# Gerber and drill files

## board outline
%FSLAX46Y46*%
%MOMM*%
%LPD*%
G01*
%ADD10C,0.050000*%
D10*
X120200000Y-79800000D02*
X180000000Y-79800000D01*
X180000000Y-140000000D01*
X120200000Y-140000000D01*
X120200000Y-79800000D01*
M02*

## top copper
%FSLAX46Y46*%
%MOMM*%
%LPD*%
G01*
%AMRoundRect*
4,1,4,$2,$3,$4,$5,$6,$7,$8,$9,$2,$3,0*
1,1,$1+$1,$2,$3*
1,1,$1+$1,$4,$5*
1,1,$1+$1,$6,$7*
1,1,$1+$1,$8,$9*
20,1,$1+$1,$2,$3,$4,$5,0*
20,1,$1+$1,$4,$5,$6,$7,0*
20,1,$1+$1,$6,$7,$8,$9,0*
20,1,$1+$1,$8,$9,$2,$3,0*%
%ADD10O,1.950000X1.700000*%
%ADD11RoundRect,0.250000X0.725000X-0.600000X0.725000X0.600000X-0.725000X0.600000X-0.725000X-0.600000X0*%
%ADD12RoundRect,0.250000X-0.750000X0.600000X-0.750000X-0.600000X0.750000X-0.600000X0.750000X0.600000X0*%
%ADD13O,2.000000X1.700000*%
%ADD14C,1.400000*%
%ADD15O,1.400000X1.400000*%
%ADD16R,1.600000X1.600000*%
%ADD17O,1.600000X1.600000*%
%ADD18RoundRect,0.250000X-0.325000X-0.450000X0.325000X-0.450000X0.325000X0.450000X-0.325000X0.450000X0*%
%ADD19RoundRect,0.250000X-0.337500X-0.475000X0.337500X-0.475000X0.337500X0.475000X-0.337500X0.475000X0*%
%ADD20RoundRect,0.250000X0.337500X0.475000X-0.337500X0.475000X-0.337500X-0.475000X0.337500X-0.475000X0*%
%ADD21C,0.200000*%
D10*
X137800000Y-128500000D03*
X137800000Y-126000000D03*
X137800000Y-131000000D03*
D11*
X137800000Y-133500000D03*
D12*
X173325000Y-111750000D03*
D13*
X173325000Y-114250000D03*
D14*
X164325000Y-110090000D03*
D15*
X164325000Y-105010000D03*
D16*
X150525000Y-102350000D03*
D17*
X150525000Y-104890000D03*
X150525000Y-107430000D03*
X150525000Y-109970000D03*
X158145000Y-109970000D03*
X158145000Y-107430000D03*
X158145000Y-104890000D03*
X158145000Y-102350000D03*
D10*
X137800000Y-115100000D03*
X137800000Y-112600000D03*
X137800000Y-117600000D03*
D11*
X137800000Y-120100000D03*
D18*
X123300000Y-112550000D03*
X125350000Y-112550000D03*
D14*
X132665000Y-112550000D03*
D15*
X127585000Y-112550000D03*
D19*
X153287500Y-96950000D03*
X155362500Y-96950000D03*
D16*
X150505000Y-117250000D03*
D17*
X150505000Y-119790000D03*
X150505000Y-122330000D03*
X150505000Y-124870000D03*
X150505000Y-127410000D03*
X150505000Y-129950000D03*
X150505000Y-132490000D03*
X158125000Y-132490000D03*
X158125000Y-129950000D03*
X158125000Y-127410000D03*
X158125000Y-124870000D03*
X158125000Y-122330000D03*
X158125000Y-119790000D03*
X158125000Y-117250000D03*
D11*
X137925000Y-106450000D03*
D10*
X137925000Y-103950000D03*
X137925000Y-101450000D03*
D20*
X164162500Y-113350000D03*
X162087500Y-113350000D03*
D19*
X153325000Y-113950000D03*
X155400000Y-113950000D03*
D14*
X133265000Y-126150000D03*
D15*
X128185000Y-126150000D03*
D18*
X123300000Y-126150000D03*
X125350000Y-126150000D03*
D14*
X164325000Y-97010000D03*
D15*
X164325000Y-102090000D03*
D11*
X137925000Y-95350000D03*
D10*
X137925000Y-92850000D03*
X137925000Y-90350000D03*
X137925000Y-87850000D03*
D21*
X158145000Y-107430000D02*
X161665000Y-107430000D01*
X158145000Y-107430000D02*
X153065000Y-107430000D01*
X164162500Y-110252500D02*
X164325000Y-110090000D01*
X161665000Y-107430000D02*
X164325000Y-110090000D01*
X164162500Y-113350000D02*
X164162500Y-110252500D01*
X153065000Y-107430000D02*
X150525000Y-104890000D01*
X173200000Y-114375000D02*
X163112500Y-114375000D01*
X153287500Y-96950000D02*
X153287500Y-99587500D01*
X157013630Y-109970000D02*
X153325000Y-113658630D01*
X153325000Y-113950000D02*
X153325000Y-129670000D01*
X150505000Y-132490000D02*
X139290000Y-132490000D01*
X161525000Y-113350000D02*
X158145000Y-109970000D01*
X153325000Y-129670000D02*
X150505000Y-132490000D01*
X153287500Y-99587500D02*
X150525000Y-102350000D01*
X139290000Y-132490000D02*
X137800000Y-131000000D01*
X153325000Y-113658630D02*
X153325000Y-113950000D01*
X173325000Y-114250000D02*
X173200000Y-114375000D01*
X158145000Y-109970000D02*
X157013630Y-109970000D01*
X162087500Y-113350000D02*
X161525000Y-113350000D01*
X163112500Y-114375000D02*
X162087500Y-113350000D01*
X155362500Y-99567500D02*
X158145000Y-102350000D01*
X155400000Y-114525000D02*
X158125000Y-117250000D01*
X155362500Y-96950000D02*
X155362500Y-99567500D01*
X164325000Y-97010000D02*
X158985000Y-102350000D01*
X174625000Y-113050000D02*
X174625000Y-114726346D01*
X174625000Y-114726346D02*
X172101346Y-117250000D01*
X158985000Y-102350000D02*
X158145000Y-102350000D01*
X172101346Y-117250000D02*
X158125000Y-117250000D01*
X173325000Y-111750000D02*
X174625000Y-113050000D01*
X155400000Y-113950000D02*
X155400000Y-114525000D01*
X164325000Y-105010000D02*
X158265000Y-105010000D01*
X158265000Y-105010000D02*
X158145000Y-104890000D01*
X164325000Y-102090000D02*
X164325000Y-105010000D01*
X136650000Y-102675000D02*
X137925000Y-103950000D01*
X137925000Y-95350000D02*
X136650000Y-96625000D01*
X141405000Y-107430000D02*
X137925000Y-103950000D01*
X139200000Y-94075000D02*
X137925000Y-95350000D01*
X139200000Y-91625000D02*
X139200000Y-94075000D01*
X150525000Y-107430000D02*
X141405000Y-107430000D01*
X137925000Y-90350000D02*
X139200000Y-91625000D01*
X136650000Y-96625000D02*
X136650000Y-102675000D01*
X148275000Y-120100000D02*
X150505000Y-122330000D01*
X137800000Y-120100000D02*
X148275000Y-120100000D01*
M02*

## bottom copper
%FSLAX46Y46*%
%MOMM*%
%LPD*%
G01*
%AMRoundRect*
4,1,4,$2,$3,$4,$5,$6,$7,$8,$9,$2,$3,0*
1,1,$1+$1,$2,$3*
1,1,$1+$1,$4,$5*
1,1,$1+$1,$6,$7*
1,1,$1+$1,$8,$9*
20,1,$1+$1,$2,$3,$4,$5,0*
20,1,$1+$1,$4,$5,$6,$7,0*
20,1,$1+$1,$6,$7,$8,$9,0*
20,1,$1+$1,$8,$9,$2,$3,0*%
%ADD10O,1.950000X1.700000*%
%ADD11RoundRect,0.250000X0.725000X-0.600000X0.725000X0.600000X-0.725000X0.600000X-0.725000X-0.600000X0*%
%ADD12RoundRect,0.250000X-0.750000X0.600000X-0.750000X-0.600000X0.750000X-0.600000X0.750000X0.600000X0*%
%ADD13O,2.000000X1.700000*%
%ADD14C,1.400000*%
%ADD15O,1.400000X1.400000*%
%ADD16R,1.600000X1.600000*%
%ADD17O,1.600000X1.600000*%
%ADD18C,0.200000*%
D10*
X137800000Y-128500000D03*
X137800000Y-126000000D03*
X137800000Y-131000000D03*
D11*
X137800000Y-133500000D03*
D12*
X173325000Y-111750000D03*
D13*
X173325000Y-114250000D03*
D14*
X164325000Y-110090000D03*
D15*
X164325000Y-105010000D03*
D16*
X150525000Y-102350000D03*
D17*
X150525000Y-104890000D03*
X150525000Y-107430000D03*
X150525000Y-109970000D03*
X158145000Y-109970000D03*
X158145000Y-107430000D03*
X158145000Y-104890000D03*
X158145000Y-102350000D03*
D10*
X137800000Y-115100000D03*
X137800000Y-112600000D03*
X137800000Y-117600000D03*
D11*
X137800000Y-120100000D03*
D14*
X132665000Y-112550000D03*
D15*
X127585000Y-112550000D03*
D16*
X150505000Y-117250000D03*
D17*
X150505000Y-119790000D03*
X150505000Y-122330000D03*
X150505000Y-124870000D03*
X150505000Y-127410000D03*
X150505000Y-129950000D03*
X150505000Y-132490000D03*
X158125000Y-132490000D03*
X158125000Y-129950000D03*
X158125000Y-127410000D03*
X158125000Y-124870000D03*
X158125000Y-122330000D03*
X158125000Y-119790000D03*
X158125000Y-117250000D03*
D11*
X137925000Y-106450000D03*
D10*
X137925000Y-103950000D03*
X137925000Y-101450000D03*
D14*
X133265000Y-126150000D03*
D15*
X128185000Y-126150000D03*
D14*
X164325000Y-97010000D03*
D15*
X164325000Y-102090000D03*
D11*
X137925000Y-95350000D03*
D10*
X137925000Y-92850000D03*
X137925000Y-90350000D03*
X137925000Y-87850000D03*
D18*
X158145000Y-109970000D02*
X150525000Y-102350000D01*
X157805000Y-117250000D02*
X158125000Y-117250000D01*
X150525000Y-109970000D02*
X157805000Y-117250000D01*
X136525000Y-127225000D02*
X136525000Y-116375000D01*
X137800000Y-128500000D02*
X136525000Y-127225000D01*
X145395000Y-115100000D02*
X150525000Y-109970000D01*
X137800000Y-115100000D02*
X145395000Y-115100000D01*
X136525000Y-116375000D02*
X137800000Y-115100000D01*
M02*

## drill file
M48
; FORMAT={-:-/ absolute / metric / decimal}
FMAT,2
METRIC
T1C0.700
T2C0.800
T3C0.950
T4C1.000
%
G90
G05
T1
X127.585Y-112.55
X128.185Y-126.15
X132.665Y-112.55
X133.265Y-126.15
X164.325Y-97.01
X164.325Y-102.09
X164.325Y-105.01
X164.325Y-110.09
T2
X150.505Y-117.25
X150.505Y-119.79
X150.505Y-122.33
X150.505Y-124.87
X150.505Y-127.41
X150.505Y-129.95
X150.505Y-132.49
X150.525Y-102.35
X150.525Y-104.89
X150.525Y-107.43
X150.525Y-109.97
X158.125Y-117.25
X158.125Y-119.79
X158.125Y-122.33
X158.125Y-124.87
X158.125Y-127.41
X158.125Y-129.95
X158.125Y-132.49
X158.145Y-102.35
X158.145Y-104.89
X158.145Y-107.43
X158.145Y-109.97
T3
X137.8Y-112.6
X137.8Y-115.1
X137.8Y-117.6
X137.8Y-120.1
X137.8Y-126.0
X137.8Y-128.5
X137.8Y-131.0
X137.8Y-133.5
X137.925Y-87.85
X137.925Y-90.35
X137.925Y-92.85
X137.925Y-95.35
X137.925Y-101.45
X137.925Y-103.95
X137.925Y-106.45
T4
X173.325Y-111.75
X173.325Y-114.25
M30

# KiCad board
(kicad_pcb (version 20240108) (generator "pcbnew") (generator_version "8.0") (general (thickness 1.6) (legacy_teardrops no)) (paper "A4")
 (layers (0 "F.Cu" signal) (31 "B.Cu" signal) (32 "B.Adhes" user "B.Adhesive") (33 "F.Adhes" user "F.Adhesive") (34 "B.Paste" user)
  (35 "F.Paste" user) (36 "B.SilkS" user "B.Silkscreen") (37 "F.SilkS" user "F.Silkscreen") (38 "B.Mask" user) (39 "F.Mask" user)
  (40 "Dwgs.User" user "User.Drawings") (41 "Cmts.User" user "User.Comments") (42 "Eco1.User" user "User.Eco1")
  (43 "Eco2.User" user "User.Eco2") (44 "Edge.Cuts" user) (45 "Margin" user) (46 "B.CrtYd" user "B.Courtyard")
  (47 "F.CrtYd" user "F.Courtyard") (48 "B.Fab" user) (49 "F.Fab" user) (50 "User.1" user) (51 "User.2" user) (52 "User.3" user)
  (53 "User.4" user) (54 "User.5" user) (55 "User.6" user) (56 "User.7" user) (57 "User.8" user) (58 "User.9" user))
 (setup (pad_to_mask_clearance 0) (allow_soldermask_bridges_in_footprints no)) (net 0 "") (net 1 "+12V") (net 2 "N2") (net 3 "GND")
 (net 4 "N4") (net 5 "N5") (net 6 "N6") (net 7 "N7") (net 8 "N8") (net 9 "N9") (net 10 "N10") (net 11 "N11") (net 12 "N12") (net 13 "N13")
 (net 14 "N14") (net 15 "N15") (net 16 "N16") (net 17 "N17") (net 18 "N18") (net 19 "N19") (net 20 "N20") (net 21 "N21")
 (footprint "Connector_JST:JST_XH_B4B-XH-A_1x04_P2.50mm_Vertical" (layer "F.Cu") (at 137.8 133.5 90)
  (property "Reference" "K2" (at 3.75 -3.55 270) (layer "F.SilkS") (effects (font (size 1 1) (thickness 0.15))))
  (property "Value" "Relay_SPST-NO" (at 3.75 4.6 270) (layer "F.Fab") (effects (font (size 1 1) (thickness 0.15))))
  (pad "13" thru_hole oval (at 5 0 90) (size 1.7 1.95) (drill 0.95) (layers "*.Cu" "*.Mask") (remove_unused_layers no) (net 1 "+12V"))
  (pad "14" thru_hole oval (at 7.5 0 90) (size 1.7 1.95) (drill 0.95) (layers "*.Cu" "*.Mask") (remove_unused_layers no) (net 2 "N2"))
  (pad "A1" thru_hole oval (at 2.5 0 90) (size 1.7 1.95) (drill 0.95) (layers "*.Cu" "*.Mask") (remove_unused_layers no) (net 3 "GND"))
  (pad "A2" thru_hole roundrect (at 0 0 90) (size 1.7 1.95) (drill 0.95) (layers "*.Cu" "*.Mask") (remove_unused_layers no)
   (roundrect_rratio 0.147059) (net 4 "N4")))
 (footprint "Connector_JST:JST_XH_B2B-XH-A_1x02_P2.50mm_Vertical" (layer "F.Cu") (at 173.325 111.75 -90)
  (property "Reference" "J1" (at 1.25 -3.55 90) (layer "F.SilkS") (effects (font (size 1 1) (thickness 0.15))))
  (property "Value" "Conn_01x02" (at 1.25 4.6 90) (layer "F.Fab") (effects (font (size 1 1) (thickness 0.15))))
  (pad "1" thru_hole roundrect (at 0 0 270) (size 1.7 2) (drill 1) (layers "*.Cu" "*.Mask") (remove_unused_layers no)
   (roundrect_rratio 0.147059) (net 1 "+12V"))
  (pad "2" thru_hole oval (at 2.5 0 270) (size 1.7 2) (drill 1) (layers "*.Cu" "*.Mask") (remove_unused_layers no) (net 3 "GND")))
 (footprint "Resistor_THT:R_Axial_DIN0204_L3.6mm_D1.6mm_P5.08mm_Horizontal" (layer "F.Cu") (at 164.325 110.09 90)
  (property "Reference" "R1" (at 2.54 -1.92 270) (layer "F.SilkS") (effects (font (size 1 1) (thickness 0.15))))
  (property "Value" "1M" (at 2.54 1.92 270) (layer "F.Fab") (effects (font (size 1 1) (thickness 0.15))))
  (pad "1" thru_hole circle (at 0 0 90) (size 1.4 1.4) (drill 0.7) (layers "*.Cu" "*.Mask") (remove_unused_layers no) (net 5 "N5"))
  (pad "2" thru_hole oval (at 5.08 0 90) (size 1.4 1.4) (drill 0.7) (layers "*.Cu" "*.Mask") (remove_unused_layers no) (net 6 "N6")))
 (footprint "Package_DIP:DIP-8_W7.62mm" (layer "F.Cu") (at 150.525 102.35)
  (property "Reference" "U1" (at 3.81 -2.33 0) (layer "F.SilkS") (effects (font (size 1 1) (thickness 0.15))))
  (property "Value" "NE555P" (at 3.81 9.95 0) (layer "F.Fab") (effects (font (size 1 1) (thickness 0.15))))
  (pad "1" thru_hole rect (at 0 0) (size 1.6 1.6) (drill 0.8) (layers "*.Cu" "*.Mask") (remove_unused_layers no) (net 3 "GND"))
  (pad "2" thru_hole oval (at 0 2.54) (size 1.6 1.6) (drill 0.8) (layers "*.Cu" "*.Mask") (remove_unused_layers no) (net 5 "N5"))
  (pad "3" thru_hole oval (at 0 5.08) (size 1.6 1.6) (drill 0.8) (layers "*.Cu" "*.Mask") (remove_unused_layers no) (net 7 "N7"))
  (pad "4" thru_hole oval (at 0 7.62) (size 1.6 1.6) (drill 0.8) (layers "*.Cu" "*.Mask") (remove_unused_layers no) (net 1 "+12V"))
  (pad "5" thru_hole oval (at 7.62 7.62) (size 1.6 1.6) (drill 0.8) (layers "*.Cu" "*.Mask") (remove_unused_layers no) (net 3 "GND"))
  (pad "6" thru_hole oval (at 7.62 5.08) (size 1.6 1.6) (drill 0.8) (layers "*.Cu" "*.Mask") (remove_unused_layers no) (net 5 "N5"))
  (pad "7" thru_hole oval (at 7.62 2.54) (size 1.6 1.6) (drill 0.8) (layers "*.Cu" "*.Mask") (remove_unused_layers no) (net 6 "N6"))
  (pad "8" thru_hole oval (at 7.62 0) (size 1.6 1.6) (drill 0.8) (layers "*.Cu" "*.Mask") (remove_unused_layers no) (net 1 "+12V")))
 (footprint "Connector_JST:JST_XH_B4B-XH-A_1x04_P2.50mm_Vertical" (layer "F.Cu") (at 137.8 120.1 90)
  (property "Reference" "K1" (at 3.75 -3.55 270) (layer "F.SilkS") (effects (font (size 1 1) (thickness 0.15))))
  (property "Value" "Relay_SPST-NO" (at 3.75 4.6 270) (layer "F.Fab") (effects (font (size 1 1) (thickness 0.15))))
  (pad "13" thru_hole oval (at 5 0 90) (size 1.7 1.95) (drill 0.95) (layers "*.Cu" "*.Mask") (remove_unused_layers no) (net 1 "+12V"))
  (pad "14" thru_hole oval (at 7.5 0 90) (size 1.7 1.95) (drill 0.95) (layers "*.Cu" "*.Mask") (remove_unused_layers no) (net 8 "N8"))
  (pad "A1" thru_hole oval (at 2.5 0 90) (size 1.7 1.95) (drill 0.95) (layers "*.Cu" "*.Mask") (remove_unused_layers no) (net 3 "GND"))
  (pad "A2" thru_hole roundrect (at 0 0 90) (size 1.7 1.95) (drill 0.95) (layers "*.Cu" "*.Mask") (remove_unused_layers no)
   (roundrect_rratio 0.147059) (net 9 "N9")))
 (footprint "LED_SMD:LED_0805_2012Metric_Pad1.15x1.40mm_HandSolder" (layer "F.Cu") (at 124.325 112.55)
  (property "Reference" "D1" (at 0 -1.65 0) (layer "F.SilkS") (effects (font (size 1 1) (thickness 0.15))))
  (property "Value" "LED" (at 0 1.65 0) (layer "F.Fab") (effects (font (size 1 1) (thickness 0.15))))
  (pad "1" smd roundrect (at -1.025 0) (size 1.15 1.4) (layers "F.Cu" "F.Paste" "F.Mask") (roundrect_rratio 0.217391) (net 3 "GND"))
  (pad "2" smd roundrect (at 1.025 0) (size 1.15 1.4) (layers "F.Cu" "F.Paste" "F.Mask") (roundrect_rratio 0.217391) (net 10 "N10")))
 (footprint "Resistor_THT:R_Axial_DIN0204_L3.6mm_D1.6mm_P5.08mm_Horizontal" (layer "F.Cu") (at 132.665 112.55 180)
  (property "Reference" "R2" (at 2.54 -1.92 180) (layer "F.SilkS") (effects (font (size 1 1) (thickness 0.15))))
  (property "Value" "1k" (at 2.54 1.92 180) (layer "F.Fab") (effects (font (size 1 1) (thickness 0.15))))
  (pad "1" thru_hole circle (at 0 0 180) (size 1.4 1.4) (drill 0.7) (layers "*.Cu" "*.Mask") (remove_unused_layers no) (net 8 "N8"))
  (pad "2" thru_hole oval (at 5.08 0 180) (size 1.4 1.4) (drill 0.7) (layers "*.Cu" "*.Mask") (remove_unused_layers no) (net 10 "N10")))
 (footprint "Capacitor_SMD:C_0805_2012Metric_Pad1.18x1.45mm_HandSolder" (layer "F.Cu") (at 154.325 96.95)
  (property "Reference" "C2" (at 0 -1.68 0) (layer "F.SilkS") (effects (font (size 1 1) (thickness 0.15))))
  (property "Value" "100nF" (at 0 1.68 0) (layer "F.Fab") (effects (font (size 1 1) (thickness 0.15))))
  (pad "1" smd roundrect (at -1.0375 0) (size 1.175 1.45) (layers "F.Cu" "F.Paste" "F.Mask") (roundrect_rratio 0.212766) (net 3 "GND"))
  (pad "2" smd roundrect (at 1.0375 0) (size 1.175 1.45) (layers "F.Cu" "F.Paste" "F.Mask") (roundrect_rratio 0.212766) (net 1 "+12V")))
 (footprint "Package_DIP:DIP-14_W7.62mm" (layer "F.Cu") (at 150.505 117.25)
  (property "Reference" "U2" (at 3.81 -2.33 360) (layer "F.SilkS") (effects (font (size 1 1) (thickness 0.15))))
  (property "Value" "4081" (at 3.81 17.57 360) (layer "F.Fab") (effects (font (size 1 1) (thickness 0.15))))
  (pad "1" thru_hole rect (at 0 0) (size 1.6 1.6) (drill 0.8) (layers "*.Cu" "*.Mask") (remove_unused_layers no) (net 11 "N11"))
  (pad "2" thru_hole oval (at 0 2.54) (size 1.6 1.6) (drill 0.8) (layers "*.Cu" "*.Mask") (remove_unused_layers no) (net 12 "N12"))
  (pad "3" thru_hole oval (at 0 5.08) (size 1.6 1.6) (drill 0.8) (layers "*.Cu" "*.Mask") (remove_unused_layers no) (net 9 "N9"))
  (pad "4" thru_hole oval (at 0 7.62) (size 1.6 1.6) (drill 0.8) (layers "*.Cu" "*.Mask") (remove_unused_layers no) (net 4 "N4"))
  (pad "5" thru_hole oval (at 0 10.16) (size 1.6 1.6) (drill 0.8) (layers "*.Cu" "*.Mask") (remove_unused_layers no) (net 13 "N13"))
  (pad "6" thru_hole oval (at 0 12.7) (size 1.6 1.6) (drill 0.8) (layers "*.Cu" "*.Mask") (remove_unused_layers no) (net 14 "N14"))
  (pad "7" thru_hole oval (at 0 15.24) (size 1.6 1.6) (drill 0.8) (layers "*.Cu" "*.Mask") (remove_unused_layers no) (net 3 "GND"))
  (pad "8" thru_hole oval (at 7.62 15.24) (size 1.6 1.6) (drill 0.8) (layers "*.Cu" "*.Mask") (remove_unused_layers no) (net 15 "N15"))
  (pad "9" thru_hole oval (at 7.62 12.7) (size 1.6 1.6) (drill 0.8) (layers "*.Cu" "*.Mask") (remove_unused_layers no) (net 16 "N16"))
  (pad "10" thru_hole oval (at 7.62 10.16) (size 1.6 1.6) (drill 0.8) (layers "*.Cu" "*.Mask") (remove_unused_layers no) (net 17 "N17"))
  (pad "11" thru_hole oval (at 7.62 7.62) (size 1.6 1.6) (drill 0.8) (layers "*.Cu" "*.Mask") (remove_unused_layers no) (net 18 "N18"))
  (pad "12" thru_hole oval (at 7.62 5.08) (size 1.6 1.6) (drill 0.8) (layers "*.Cu" "*.Mask") (remove_unused_layers no) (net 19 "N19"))
  (pad "13" thru_hole oval (at 7.62 2.54) (size 1.6 1.6) (drill 0.8) (layers "*.Cu" "*.Mask") (remove_unused_layers no) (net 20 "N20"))
  (pad "14" thru_hole oval (at 7.62 0) (size 1.6 1.6) (drill 0.8) (layers "*.Cu" "*.Mask") (remove_unused_layers no) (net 1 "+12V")))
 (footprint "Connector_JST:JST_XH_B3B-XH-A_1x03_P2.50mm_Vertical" (layer "F.Cu") (at 137.925 106.45 90)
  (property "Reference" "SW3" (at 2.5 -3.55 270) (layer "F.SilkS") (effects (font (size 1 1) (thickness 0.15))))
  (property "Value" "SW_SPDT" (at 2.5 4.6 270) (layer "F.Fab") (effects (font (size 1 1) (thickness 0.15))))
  (pad "1" thru_hole roundrect (at 0 0 90) (size 1.7 1.95) (drill 0.95) (layers "*.Cu" "*.Mask") (remove_unused_layers no)
   (roundrect_rratio 0.147059) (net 11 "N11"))
  (pad "2" thru_hole oval (at 2.5 0 90) (size 1.7 1.95) (drill 0.95) (layers "*.Cu" "*.Mask") (remove_unused_layers no) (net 7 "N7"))
  (pad "3" thru_hole oval (at 5 0 90) (size 1.7 1.95) (drill 0.95) (layers "*.Cu" "*.Mask") (remove_unused_layers no) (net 13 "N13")))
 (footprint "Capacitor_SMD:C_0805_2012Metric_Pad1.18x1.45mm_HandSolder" (layer "F.Cu") (at 163.125 113.35 180)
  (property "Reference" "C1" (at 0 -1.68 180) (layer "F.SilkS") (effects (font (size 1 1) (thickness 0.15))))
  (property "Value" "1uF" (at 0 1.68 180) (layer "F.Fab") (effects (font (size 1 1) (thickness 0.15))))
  (pad "1" smd roundrect (at -1.0375 0 180) (size 1.175 1.45) (layers "F.Cu" "F.Paste" "F.Mask") (roundrect_rratio 0.212766) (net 5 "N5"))
  (pad "2" smd roundrect (at 1.0375 0 180) (size 1.175 1.45) (layers "F.Cu" "F.Paste" "F.Mask") (roundrect_rratio 0.212766) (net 3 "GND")))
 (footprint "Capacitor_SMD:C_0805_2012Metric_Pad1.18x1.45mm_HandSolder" (layer "F.Cu") (at 154.3625 113.95)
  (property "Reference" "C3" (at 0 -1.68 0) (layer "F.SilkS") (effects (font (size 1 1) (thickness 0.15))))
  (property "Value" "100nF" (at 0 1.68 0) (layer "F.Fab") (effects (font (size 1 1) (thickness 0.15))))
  (pad "1" smd roundrect (at -1.0375 0) (size 1.175 1.45) (layers "F.Cu" "F.Paste" "F.Mask") (roundrect_rratio 0.212766) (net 3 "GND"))
  (pad "2" smd roundrect (at 1.0375 0) (size 1.175 1.45) (layers "F.Cu" "F.Paste" "F.Mask") (roundrect_rratio 0.212766) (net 1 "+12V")))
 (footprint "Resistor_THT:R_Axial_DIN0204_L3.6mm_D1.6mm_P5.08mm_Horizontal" (layer "F.Cu") (at 133.265 126.15 180)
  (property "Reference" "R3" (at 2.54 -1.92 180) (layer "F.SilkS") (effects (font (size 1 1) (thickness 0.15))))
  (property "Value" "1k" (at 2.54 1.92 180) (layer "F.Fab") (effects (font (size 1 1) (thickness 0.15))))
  (pad "1" thru_hole circle (at 0 0 180) (size 1.4 1.4) (drill 0.7) (layers "*.Cu" "*.Mask") (remove_unused_layers no) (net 2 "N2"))
  (pad "2" thru_hole oval (at 5.08 0 180) (size 1.4 1.4) (drill 0.7) (layers "*.Cu" "*.Mask") (remove_unused_layers no) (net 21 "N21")))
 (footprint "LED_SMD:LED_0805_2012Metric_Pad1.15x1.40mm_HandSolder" (layer "F.Cu") (at 124.325 126.15)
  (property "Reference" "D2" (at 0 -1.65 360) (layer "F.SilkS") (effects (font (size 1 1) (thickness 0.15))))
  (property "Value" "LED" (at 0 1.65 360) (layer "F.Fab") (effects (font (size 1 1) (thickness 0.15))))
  (pad "1" smd roundrect (at -1.025 0) (size 1.15 1.4) (layers "F.Cu" "F.Paste" "F.Mask") (roundrect_rratio 0.217391) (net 3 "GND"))
  (pad "2" smd roundrect (at 1.025 0) (size 1.15 1.4) (layers "F.Cu" "F.Paste" "F.Mask") (roundrect_rratio 0.217391) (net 21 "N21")))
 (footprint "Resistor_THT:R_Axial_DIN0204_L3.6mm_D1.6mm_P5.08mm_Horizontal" (layer "F.Cu") (at 164.325 97.01 -90)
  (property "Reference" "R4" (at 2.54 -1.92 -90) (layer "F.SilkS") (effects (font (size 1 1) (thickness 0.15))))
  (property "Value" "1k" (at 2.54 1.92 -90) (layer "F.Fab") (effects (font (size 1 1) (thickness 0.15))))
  (pad "1" thru_hole circle (at 0 0 270) (size 1.4 1.4) (drill 0.7) (layers "*.Cu" "*.Mask") (remove_unused_layers no) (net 1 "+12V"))
  (pad "2" thru_hole oval (at 5.08 0 270) (size 1.4 1.4) (drill 0.7) (layers "*.Cu" "*.Mask") (remove_unused_layers no) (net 6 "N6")))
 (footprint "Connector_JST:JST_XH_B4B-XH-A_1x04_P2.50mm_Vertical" (layer "F.Cu") (at 137.925 95.35 90)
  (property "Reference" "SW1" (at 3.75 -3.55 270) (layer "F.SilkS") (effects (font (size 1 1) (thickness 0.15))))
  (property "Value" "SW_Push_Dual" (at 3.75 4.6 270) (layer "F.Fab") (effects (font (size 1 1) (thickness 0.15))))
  (pad "1" thru_hole roundrect (at 0 0 90) (size 1.7 1.95) (drill 0.95) (layers "*.Cu" "*.Mask") (remove_unused_layers no)
   (roundrect_rratio 0.147059) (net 7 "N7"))
  (pad "2" thru_hole oval (at 2.5 0 90) (size 1.7 1.95) (drill 0.95) (layers "*.Cu" "*.Mask") (remove_unused_layers no) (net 12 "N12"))
  (pad "3" thru_hole oval (at 5 0 90) (size 1.7 1.95) (drill 0.95) (layers "*.Cu" "*.Mask") (remove_unused_layers no) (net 7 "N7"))
  (pad "4" thru_hole oval (at 7.5 0 90) (size 1.7 1.95) (drill 0.95) (layers "*.Cu" "*.Mask") (remove_unused_layers no) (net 14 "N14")))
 (gr_rect (start 120.2 79.8) (end 180 140) (stroke (width 0.05) (type default)) (fill none) (layer "Edge.Cuts"))
 (segment (start 158.145 107.43) (end 161.665 107.43) (width 0.2) (layer "F.Cu") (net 5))
 (segment (start 158.145 107.43) (end 153.065 107.43) (width 0.2) (layer "F.Cu") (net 5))
 (segment (start 164.1625 110.2525) (end 164.325 110.09) (width 0.2) (layer "F.Cu") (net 5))
 (segment (start 161.665 107.43) (end 164.325 110.09) (width 0.2) (layer "F.Cu") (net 5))
 (segment (start 164.1625 113.35) (end 164.1625 110.2525) (width 0.2) (layer "F.Cu") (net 5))
 (segment (start 153.065 107.43) (end 150.525 104.89) (width 0.2) (layer "F.Cu") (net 5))
 (segment (start 173.2 114.375) (end 163.1125 114.375) (width 0.2) (layer "F.Cu") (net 3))
 (segment (start 153.2875 96.95) (end 153.2875 99.5875) (width 0.2) (layer "F.Cu") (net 3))
 (segment (start 157.01363 109.97) (end 153.325 113.65863) (width 0.2) (layer "F.Cu") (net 3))
 (segment (start 153.325 113.95) (end 153.325 129.67) (width 0.2) (layer "F.Cu") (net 3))
 (segment (start 150.505 132.49) (end 139.29 132.49) (width 0.2) (layer "F.Cu") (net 3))
 (segment (start 161.525 113.35) (end 158.145 109.97) (width 0.2) (layer "F.Cu") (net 3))
 (segment (start 153.325 129.67) (end 150.505 132.49) (width 0.2) (layer "F.Cu") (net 3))
 (segment (start 153.2875 99.5875) (end 150.525 102.35) (width 0.2) (layer "F.Cu") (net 3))
 (segment (start 139.29 132.49) (end 137.8 131) (width 0.2) (layer "F.Cu") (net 3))
 (segment (start 153.325 113.65863) (end 153.325 113.95) (width 0.2) (layer "F.Cu") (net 3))
 (segment (start 173.325 114.25) (end 173.2 114.375) (width 0.2) (layer "F.Cu") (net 3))
 (segment (start 158.145 109.97) (end 157.01363 109.97) (width 0.2) (layer "F.Cu") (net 3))
 (segment (start 162.0875 113.35) (end 161.525 113.35) (width 0.2) (layer "F.Cu") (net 3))
 (segment (start 163.1125 114.375) (end 162.0875 113.35) (width 0.2) (layer "F.Cu") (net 3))
 (segment (start 158.145 109.97) (end 150.525 102.35) (width 0.2) (layer "B.Cu") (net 3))
 (segment (start 155.3625 99.5675) (end 158.145 102.35) (width 0.2) (layer "F.Cu") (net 1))
 (segment (start 155.4 114.525) (end 158.125 117.25) (width 0.2) (layer "F.Cu") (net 1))
 (segment (start 155.3625 96.95) (end 155.3625 99.5675) (width 0.2) (layer "F.Cu") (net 1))
 (segment (start 164.325 97.01) (end 158.985 102.35) (width 0.2) (layer "F.Cu") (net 1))
 (segment (start 174.625 113.05) (end 174.625 114.726346) (width 0.2) (layer "F.Cu") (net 1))
 (segment (start 174.625 114.726346) (end 172.101346 117.25) (width 0.2) (layer "F.Cu") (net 1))
 (segment (start 158.985 102.35) (end 158.145 102.35) (width 0.2) (layer "F.Cu") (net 1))
 (segment (start 172.101346 117.25) (end 158.125 117.25) (width 0.2) (layer "F.Cu") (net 1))
 (segment (start 173.325 111.75) (end 174.625 113.05) (width 0.2) (layer "F.Cu") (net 1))
 (segment (start 155.4 113.95) (end 155.4 114.525) (width 0.2) (layer "F.Cu") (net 1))
 (segment (start 157.805 117.25) (end 158.125 117.25) (width 0.2) (layer "B.Cu") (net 1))
 (segment (start 150.525 109.97) (end 157.805 117.25) (width 0.2) (layer "B.Cu") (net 1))
 (segment (start 136.525 127.225) (end 136.525 116.375) (width 0.2) (layer "B.Cu") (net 1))
 (segment (start 137.8 128.5) (end 136.525 127.225) (width 0.2) (layer "B.Cu") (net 1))
 (segment (start 145.395 115.1) (end 150.525 109.97) (width 0.2) (layer "B.Cu") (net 1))
 (segment (start 137.8 115.1) (end 145.395 115.1) (width 0.2) (layer "B.Cu") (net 1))
 (segment (start 136.525 116.375) (end 137.8 115.1) (width 0.2) (layer "B.Cu") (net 1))
 (segment (start 164.325 105.01) (end 158.265 105.01) (width 0.2) (layer "F.Cu") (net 6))
 (segment (start 158.265 105.01) (end 158.145 104.89) (width 0.2) (layer "F.Cu") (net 6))
 (segment (start 164.325 102.09) (end 164.325 105.01) (width 0.2) (layer "F.Cu") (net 6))
 (segment (start 136.65 102.675) (end 137.925 103.95) (width 0.2) (layer "F.Cu") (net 7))
 (segment (start 137.925 95.35) (end 136.65 96.625) (width 0.2) (layer "F.Cu") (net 7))
 (segment (start 141.405 107.43) (end 137.925 103.95) (width 0.2) (layer "F.Cu") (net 7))
 (segment (start 139.2 94.075) (end 137.925 95.35) (width 0.2) (layer "F.Cu") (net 7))
 (segment (start 139.2 91.625) (end 139.2 94.075) (width 0.2) (layer "F.Cu") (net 7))
 (segment (start 150.525 107.43) (end 141.405 107.43) (width 0.2) (layer "F.Cu") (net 7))
 (segment (start 137.925 90.35) (end 139.2 91.625) (width 0.2) (layer "F.Cu") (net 7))
 (segment (start 136.65 96.625) (end 136.65 102.675) (width 0.2) (layer "F.Cu") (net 7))
 (segment (start 148.275 120.1) (end 150.505 122.33) (width 0.2) (layer "F.Cu") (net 9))
 (segment (start 137.8 120.1) (end 148.275 120.1) (width 0.2) (layer "F.Cu") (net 9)))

